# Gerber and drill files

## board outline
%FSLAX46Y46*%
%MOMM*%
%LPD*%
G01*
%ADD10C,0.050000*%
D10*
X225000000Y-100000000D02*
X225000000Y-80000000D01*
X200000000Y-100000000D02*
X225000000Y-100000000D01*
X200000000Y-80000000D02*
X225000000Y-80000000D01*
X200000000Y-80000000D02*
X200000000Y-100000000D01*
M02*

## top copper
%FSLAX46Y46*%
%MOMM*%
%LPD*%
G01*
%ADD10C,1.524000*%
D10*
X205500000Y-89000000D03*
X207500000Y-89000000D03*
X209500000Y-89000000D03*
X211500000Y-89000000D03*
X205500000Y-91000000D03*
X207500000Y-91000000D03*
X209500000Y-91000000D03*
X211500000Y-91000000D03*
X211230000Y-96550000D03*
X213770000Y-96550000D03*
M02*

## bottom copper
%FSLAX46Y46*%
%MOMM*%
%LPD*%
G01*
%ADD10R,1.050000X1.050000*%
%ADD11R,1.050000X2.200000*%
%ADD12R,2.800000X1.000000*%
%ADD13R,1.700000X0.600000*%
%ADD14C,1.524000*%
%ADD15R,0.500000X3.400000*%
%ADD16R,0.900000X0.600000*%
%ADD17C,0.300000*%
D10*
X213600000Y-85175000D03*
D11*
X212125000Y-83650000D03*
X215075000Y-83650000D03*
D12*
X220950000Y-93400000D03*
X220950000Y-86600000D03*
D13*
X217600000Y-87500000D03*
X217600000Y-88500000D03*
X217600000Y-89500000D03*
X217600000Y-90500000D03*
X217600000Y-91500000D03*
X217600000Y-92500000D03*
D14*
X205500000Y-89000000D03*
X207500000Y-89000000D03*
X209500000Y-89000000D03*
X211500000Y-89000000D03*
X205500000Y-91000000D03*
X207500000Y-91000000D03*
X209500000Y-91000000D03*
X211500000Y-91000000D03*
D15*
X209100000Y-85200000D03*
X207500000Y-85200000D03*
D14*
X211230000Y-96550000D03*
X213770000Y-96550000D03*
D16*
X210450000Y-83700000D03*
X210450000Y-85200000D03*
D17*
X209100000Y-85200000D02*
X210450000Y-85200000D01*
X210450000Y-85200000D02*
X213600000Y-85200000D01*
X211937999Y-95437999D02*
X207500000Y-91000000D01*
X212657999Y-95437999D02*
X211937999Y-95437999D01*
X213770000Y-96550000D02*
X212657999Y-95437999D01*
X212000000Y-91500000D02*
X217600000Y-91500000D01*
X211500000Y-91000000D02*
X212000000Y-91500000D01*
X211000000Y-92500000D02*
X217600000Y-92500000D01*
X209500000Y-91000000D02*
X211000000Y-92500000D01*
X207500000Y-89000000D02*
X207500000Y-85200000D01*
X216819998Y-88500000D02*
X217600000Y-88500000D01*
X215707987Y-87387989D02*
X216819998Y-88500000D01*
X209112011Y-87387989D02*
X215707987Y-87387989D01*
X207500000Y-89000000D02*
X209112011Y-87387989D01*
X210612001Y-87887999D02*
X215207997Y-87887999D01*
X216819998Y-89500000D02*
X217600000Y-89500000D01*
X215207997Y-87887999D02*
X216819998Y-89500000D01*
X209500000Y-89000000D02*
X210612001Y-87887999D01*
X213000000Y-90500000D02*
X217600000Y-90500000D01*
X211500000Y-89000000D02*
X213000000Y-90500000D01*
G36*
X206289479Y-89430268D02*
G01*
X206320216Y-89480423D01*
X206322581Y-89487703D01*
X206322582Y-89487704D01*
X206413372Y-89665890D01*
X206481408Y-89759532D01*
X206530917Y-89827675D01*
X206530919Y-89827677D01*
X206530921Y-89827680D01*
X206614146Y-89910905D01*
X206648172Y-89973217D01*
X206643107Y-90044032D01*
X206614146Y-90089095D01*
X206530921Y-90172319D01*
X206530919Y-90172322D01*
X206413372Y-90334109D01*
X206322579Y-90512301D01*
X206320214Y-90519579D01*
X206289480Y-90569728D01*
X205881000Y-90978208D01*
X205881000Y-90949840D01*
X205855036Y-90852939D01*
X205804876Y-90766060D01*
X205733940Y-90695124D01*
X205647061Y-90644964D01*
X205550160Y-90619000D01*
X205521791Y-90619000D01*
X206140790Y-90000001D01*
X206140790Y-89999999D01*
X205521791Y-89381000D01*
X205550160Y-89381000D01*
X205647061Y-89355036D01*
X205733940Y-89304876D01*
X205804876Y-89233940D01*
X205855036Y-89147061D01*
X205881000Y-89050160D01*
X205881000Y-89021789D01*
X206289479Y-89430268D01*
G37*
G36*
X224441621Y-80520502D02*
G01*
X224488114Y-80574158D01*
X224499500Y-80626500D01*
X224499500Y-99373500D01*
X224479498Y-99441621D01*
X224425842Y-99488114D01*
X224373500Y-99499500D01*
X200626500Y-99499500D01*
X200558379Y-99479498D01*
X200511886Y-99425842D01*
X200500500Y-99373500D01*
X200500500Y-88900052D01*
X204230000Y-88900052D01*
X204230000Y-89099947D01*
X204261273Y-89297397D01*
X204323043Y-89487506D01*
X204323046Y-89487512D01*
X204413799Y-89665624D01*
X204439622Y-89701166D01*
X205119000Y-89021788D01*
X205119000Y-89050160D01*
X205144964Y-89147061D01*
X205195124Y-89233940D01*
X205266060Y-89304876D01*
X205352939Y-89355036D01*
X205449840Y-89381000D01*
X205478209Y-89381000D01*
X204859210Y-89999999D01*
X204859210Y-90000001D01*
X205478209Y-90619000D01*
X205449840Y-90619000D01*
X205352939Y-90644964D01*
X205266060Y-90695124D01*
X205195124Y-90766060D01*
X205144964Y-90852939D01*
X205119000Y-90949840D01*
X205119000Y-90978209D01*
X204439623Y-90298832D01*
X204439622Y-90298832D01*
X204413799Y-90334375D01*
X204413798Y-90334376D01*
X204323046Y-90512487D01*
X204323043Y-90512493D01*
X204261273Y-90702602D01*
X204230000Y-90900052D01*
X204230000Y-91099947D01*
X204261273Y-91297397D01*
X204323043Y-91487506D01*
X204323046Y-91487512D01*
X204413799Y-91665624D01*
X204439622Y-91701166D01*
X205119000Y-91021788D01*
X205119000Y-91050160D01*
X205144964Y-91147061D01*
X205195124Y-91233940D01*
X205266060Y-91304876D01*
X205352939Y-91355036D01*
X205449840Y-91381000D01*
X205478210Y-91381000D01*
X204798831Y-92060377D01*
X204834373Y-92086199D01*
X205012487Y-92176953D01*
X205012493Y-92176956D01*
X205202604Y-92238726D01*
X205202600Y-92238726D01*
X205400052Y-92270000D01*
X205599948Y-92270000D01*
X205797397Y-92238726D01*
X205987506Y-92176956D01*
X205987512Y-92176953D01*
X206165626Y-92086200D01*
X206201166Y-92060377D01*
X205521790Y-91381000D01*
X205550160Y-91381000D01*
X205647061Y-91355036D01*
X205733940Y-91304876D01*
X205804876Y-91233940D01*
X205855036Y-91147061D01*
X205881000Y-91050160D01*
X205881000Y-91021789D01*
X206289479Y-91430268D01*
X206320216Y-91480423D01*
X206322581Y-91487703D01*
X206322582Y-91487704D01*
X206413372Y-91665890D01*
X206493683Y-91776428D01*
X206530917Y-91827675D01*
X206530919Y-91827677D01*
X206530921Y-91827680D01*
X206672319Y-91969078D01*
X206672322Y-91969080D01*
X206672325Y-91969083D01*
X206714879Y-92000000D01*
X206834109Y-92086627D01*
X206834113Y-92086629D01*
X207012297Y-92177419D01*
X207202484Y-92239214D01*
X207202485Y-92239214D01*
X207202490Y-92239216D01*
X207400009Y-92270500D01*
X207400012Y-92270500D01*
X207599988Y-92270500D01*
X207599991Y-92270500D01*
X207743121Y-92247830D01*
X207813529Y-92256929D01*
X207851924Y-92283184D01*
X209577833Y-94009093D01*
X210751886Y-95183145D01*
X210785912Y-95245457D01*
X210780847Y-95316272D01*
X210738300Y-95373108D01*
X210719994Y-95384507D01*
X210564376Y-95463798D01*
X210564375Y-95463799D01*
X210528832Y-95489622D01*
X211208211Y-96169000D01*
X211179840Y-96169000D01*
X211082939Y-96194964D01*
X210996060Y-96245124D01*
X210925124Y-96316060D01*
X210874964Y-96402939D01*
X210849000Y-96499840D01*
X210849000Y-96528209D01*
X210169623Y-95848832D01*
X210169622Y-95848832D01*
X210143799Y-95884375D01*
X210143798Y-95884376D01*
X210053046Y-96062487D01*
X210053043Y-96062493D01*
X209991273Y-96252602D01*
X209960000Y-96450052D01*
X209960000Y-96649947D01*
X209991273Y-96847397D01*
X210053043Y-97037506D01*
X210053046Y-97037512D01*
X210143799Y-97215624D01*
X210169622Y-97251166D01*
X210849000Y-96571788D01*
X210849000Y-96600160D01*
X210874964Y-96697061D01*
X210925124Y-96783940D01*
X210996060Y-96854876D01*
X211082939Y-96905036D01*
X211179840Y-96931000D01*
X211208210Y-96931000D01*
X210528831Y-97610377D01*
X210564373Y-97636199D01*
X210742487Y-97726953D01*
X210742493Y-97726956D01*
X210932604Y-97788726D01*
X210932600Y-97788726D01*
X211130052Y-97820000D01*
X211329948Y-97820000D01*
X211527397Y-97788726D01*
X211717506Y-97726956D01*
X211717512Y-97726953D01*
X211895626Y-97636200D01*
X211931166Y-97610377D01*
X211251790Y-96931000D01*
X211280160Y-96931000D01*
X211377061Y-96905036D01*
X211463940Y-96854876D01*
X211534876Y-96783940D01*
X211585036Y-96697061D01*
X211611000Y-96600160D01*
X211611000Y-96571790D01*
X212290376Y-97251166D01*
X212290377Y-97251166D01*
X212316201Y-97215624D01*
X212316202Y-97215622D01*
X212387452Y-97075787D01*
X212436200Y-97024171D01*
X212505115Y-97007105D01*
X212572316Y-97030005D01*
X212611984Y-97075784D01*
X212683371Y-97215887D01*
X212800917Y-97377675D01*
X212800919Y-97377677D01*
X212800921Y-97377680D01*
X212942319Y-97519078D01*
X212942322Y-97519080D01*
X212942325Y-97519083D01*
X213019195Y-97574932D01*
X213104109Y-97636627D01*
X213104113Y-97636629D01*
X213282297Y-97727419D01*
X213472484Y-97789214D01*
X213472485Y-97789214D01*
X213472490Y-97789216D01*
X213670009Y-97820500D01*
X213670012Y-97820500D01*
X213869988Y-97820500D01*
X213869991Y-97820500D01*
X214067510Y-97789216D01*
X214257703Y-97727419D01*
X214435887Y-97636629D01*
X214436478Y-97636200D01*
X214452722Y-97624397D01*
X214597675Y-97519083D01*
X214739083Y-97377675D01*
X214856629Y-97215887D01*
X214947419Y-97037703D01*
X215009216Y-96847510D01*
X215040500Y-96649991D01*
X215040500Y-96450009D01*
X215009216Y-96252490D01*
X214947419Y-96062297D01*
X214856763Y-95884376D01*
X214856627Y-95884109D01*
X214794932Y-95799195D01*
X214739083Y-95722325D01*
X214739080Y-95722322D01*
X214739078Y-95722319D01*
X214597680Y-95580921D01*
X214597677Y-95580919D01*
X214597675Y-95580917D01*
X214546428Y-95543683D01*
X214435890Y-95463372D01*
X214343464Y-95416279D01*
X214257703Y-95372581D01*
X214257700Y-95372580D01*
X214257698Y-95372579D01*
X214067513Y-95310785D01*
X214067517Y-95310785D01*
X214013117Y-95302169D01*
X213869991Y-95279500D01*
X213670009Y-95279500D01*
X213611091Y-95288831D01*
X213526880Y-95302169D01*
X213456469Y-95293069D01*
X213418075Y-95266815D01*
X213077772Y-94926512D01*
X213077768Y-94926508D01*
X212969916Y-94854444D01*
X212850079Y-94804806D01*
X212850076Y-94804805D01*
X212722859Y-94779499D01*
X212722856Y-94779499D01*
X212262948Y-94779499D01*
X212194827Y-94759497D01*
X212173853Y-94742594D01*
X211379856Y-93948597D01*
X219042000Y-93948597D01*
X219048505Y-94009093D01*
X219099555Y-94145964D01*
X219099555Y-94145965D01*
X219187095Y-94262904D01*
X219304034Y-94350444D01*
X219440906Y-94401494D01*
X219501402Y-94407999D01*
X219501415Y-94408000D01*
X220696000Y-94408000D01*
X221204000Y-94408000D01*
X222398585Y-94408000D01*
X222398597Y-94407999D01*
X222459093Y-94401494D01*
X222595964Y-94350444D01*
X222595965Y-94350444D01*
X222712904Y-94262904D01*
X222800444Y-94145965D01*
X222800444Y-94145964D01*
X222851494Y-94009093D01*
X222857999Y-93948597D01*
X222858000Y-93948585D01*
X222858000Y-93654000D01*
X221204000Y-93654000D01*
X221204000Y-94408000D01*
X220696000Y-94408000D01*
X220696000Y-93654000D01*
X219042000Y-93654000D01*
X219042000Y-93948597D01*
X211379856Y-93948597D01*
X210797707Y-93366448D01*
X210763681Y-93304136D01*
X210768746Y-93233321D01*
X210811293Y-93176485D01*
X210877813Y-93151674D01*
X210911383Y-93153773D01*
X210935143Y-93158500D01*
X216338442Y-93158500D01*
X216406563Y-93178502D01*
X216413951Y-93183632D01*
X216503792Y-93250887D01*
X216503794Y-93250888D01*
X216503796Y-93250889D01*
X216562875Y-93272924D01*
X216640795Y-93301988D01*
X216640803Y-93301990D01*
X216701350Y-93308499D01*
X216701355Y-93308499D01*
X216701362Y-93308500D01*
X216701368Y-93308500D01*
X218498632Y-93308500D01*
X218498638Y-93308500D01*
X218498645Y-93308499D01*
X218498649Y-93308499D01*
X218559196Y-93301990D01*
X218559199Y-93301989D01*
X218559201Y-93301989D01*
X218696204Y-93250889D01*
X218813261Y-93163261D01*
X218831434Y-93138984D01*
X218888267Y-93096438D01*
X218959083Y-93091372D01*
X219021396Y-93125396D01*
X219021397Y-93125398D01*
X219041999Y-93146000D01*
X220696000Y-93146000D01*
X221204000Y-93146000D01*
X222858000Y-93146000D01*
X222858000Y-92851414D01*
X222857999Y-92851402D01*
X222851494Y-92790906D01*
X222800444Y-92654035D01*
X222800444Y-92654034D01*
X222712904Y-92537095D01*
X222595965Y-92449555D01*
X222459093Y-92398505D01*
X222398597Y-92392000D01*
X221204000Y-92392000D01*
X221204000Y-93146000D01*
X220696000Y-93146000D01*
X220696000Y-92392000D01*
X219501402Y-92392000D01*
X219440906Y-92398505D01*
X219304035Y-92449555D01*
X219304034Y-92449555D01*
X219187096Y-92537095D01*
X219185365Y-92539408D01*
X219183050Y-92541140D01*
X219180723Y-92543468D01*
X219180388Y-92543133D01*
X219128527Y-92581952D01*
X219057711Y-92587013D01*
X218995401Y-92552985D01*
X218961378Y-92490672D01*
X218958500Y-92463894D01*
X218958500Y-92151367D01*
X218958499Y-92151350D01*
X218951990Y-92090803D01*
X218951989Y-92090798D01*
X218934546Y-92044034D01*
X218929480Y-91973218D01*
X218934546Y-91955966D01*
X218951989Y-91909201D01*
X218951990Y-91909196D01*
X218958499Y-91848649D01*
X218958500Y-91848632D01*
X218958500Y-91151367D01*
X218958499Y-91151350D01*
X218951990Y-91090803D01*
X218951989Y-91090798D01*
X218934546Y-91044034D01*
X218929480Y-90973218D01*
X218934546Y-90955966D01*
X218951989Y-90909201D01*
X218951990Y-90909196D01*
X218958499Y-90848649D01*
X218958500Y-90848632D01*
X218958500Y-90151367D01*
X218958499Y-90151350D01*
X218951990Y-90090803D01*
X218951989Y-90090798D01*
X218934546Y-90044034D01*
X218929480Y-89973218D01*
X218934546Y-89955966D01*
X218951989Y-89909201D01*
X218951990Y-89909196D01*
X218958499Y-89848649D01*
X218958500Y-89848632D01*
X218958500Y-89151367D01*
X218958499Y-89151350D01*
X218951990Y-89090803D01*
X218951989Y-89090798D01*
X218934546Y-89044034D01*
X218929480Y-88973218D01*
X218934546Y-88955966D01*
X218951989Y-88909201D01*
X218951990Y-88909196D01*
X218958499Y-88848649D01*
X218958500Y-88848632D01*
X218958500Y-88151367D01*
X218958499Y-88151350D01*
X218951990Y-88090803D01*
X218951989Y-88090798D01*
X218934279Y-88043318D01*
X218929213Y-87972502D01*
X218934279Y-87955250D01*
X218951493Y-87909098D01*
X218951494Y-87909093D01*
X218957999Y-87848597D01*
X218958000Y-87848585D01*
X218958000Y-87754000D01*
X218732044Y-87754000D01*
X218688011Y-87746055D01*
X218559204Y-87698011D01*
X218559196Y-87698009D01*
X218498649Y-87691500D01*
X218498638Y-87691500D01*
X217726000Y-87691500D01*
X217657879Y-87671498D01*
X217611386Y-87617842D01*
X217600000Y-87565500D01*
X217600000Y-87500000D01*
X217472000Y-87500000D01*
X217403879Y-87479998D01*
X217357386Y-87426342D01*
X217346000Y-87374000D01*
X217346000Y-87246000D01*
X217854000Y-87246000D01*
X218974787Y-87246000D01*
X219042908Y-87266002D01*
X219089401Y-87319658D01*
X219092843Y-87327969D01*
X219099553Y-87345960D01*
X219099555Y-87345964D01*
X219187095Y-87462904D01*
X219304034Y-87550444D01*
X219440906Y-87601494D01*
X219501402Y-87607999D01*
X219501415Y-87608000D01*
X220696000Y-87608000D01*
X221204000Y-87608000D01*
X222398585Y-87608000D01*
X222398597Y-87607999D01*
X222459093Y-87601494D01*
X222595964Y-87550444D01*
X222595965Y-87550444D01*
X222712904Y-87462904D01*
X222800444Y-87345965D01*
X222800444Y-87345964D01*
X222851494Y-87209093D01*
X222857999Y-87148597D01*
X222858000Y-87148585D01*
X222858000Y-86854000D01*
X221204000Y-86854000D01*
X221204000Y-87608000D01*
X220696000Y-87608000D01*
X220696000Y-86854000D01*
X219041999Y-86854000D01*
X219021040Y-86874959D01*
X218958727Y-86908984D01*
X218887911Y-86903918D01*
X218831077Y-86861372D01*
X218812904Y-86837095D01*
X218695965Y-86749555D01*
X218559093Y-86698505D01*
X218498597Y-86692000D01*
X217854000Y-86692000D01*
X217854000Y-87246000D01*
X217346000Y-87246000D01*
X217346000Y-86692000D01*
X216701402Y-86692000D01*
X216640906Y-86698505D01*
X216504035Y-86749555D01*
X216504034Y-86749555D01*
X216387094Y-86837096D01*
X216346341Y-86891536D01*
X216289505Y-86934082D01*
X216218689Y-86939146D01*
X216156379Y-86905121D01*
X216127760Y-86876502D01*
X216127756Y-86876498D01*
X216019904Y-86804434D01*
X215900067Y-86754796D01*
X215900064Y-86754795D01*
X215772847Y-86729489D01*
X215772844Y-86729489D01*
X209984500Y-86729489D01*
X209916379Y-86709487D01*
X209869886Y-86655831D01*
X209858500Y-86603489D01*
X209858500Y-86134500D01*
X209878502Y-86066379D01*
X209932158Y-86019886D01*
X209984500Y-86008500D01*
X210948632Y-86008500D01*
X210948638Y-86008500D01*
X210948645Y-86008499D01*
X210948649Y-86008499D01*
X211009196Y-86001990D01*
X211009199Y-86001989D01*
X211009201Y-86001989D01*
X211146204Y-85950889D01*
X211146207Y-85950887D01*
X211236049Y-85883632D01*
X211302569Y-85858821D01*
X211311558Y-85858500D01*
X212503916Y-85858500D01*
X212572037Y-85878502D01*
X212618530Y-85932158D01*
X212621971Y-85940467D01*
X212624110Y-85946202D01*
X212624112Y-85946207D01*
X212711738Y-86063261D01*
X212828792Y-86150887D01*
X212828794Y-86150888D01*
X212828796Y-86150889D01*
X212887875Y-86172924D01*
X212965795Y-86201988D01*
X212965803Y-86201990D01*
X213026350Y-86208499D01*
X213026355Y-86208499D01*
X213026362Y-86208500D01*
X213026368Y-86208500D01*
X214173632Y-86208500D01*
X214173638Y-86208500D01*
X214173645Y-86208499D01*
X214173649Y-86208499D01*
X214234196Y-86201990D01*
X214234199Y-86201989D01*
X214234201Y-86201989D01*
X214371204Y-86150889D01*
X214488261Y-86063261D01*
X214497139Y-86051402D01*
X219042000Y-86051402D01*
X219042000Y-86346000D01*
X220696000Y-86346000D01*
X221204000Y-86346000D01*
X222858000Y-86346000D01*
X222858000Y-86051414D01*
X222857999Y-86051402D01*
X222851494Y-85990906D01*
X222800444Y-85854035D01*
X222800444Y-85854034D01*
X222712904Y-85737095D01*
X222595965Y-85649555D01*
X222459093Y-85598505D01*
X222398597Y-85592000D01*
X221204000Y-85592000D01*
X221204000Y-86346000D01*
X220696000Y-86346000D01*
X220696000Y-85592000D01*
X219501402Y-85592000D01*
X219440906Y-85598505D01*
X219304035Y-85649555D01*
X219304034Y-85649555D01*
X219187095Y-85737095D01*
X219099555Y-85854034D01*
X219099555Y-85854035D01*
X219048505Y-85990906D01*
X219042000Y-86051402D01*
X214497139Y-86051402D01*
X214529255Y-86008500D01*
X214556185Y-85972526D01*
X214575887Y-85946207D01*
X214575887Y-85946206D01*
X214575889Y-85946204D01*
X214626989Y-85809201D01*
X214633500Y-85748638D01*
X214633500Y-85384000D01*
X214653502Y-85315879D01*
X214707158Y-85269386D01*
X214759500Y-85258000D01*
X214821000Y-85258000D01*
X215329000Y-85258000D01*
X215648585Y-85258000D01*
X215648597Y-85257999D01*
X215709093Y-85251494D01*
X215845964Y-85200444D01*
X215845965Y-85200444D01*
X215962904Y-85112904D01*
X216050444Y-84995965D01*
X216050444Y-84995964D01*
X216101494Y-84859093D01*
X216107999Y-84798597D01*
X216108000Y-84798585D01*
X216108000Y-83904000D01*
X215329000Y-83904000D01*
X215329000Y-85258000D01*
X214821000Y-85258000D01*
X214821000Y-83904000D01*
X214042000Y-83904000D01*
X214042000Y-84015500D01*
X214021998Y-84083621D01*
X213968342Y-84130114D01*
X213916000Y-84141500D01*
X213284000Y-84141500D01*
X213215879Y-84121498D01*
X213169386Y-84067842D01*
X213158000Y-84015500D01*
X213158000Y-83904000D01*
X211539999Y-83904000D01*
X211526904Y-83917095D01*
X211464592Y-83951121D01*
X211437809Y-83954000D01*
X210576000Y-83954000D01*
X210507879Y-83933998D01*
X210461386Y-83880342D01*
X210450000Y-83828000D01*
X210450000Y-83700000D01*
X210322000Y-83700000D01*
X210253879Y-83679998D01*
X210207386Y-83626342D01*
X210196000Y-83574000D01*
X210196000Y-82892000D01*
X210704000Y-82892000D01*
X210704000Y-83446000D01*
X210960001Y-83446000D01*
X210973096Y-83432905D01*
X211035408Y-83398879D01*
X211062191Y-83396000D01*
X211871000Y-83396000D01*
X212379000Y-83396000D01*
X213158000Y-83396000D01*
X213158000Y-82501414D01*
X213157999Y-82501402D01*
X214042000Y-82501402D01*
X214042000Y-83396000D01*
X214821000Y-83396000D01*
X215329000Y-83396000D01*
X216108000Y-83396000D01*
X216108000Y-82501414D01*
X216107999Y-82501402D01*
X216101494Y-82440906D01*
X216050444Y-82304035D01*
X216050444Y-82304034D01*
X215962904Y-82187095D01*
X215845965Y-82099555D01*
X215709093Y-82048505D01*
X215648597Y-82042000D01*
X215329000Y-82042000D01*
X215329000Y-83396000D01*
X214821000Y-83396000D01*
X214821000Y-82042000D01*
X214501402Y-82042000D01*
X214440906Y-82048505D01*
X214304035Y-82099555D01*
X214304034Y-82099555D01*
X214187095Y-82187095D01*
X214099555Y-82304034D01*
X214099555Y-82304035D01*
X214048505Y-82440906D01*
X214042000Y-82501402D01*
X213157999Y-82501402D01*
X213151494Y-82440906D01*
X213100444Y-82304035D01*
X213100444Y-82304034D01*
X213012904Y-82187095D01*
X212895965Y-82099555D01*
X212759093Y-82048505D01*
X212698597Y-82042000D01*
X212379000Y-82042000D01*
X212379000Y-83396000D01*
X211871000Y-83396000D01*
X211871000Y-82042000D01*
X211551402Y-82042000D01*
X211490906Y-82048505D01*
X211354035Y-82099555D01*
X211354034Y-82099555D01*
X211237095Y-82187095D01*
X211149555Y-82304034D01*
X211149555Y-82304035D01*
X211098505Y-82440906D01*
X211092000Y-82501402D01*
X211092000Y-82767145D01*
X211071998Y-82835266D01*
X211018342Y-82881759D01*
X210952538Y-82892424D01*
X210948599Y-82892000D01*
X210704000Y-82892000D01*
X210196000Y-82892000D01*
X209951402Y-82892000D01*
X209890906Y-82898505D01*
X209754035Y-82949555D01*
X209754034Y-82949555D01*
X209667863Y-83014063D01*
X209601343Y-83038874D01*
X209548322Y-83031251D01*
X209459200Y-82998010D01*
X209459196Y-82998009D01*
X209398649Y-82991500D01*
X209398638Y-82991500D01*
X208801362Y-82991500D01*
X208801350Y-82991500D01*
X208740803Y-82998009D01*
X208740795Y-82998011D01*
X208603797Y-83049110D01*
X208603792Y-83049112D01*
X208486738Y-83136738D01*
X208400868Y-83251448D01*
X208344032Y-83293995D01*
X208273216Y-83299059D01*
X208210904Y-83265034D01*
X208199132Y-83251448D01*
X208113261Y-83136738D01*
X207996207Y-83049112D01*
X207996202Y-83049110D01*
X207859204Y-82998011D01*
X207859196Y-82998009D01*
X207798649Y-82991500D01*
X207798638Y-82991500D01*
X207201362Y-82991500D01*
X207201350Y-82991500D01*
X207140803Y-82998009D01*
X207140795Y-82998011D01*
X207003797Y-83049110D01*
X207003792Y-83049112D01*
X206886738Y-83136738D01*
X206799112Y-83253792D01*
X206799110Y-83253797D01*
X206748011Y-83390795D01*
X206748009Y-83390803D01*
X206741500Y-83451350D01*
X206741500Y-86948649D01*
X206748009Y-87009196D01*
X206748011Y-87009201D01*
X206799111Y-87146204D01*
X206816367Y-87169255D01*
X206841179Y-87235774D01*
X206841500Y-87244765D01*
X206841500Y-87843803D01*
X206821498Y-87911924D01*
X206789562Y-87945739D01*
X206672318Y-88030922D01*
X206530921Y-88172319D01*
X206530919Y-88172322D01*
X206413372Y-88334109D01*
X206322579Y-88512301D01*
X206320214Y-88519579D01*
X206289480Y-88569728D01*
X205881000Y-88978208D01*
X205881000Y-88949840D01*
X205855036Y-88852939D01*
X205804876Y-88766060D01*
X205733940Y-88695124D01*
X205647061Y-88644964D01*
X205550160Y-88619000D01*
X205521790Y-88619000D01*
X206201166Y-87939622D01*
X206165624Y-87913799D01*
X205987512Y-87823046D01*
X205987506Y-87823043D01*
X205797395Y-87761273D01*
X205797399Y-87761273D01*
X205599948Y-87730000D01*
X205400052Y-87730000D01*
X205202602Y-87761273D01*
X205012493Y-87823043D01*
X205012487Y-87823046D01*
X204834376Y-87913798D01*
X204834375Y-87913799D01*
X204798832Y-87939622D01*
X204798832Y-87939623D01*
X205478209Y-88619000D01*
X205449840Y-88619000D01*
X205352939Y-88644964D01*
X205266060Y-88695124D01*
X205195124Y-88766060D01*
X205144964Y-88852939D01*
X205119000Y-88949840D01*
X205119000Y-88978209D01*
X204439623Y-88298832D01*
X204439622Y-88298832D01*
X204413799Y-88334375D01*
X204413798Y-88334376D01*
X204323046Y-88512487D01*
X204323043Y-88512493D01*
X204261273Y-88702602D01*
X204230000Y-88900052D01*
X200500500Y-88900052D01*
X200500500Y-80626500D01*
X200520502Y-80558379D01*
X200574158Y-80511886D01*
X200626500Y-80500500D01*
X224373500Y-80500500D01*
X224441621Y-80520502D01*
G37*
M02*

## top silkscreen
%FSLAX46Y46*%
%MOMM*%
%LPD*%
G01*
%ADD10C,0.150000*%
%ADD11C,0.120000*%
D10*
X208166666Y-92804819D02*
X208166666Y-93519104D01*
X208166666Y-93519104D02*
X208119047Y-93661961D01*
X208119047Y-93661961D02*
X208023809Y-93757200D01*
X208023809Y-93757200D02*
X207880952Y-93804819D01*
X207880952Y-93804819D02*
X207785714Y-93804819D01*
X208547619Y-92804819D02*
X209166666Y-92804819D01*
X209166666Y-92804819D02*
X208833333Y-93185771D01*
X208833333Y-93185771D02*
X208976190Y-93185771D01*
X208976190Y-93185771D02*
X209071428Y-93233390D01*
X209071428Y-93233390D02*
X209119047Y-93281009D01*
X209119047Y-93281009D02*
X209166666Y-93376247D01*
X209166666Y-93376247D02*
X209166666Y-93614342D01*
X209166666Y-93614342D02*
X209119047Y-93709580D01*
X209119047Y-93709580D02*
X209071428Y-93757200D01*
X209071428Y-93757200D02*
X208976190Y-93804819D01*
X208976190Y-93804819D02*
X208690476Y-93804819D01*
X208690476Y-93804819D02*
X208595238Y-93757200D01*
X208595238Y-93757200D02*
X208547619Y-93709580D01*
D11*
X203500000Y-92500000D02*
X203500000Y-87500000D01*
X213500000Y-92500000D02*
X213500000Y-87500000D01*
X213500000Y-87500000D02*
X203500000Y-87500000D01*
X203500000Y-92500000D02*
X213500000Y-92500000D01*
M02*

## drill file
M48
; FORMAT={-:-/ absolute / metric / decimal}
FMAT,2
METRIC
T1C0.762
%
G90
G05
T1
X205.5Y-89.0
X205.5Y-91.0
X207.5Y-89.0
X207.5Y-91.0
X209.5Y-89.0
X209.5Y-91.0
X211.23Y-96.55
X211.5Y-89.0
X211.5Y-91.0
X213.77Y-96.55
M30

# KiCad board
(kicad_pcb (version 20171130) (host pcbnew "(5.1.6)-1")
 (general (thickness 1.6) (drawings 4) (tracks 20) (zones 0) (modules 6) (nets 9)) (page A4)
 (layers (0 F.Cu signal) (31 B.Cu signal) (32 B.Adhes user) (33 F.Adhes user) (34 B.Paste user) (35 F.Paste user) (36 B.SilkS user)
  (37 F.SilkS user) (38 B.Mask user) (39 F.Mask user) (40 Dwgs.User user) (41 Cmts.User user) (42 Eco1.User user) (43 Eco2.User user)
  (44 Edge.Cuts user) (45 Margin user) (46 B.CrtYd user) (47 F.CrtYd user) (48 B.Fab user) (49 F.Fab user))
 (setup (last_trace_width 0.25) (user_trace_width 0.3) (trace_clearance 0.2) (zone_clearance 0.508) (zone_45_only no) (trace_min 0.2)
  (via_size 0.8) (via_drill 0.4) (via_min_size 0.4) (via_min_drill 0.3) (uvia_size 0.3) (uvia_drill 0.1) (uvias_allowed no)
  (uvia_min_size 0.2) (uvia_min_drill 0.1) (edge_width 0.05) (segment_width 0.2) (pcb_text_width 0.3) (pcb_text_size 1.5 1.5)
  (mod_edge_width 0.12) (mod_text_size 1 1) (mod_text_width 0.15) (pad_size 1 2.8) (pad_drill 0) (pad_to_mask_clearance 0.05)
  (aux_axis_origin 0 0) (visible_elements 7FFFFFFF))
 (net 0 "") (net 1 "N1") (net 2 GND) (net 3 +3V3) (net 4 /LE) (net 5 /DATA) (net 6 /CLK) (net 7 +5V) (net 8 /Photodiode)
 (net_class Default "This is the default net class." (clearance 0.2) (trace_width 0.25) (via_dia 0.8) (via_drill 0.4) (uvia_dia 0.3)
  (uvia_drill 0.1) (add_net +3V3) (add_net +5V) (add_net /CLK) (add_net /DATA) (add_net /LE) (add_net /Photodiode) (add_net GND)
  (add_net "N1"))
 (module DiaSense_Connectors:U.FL (layer B.Cu) (at 213.6 83.65 180)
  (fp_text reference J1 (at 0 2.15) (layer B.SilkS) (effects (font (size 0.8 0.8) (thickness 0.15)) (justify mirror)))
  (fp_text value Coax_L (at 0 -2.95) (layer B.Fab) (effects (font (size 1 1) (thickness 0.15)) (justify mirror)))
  (pad 1 smd rect (at 0 -1.525 180) (size 1.05 1.05) (layers B.Cu B.Paste B.Mask) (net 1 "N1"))
  (pad 2 smd rect (at 1.475 0 180) (size 1.05 2.2) (layers B.Cu B.Paste B.Mask) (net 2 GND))
  (pad 2 smd rect (at -1.475 0 180) (size 1.05 2.2) (layers B.Cu B.Paste B.Mask) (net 2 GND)))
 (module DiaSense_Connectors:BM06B (layer B.Cu) (at 218.45 90 90)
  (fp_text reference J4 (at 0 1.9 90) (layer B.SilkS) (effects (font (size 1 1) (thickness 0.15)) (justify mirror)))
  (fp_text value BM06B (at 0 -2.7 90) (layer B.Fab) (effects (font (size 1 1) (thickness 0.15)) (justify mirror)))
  (pad "" smd rect (at -3.4 2.5 90) (size 1 2.8) (layers B.Cu B.Paste B.Mask) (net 2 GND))
  (pad "" smd rect (at 3.4 2.5 90) (size 1 2.8) (layers B.Cu B.Paste B.Mask) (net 2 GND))
  (pad 6 smd rect (at 2.5 -0.85 90) (size 0.6 1.7) (layers B.Cu B.Paste B.Mask) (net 2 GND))
  (pad 5 smd rect (at 1.5 -0.85 90) (size 0.6 1.7) (layers B.Cu B.Paste B.Mask) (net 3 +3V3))
  (pad 4 smd rect (at 0.5 -0.85 90) (size 0.6 1.7) (layers B.Cu B.Paste B.Mask) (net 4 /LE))
  (pad 3 smd rect (at -0.5 -0.85 90) (size 0.6 1.7) (layers B.Cu B.Paste B.Mask) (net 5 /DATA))
  (pad 2 smd rect (at -1.5 -0.85 90) (size 0.6 1.7) (layers B.Cu B.Paste B.Mask) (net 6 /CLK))
  (pad 1 smd rect (at -2.5 -0.85 90) (size 0.6 1.7) (layers B.Cu B.Paste B.Mask) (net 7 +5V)))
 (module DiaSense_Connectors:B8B (layer F.Cu) (at 208.5 90 180)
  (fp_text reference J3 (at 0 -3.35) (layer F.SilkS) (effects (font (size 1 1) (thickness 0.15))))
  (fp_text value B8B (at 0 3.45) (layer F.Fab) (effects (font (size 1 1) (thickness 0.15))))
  (fp_line (start 5 -2.5) (end 5 2.5) (layer F.SilkS) (width 0.12))
  (fp_line (start -5 -2.5) (end -5 2.5) (layer F.SilkS) (width 0.12))
  (fp_line (start -5 2.5) (end 5 2.5) (layer F.SilkS) (width 0.12))
  (fp_line (start 5 -2.5) (end -5 -2.5) (layer F.SilkS) (width 0.12))
  (pad 8 thru_hole circle (at 3 1 180) (size 1.524 1.524) (drill 0.762) (layers *.Cu *.Mask) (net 2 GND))
  (pad 7 thru_hole circle (at 1 1 180) (size 1.524 1.524) (drill 0.762) (layers *.Cu *.Mask) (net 3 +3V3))
  (pad 6 thru_hole circle (at -1 1 180) (size 1.524 1.524) (drill 0.762) (layers *.Cu *.Mask) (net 4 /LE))
  (pad 5 thru_hole circle (at -3 1 180) (size 1.524 1.524) (drill 0.762) (layers *.Cu *.Mask) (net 5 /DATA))
  (pad 4 thru_hole circle (at 3 -1 180) (size 1.524 1.524) (drill 0.762) (layers *.Cu *.Mask) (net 2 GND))
  (pad 3 thru_hole circle (at 1 -1 180) (size 1.524 1.524) (drill 0.762) (layers *.Cu *.Mask) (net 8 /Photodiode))
  (pad 2 thru_hole circle (at -1 -1 180) (size 1.524 1.524) (drill 0.762) (layers *.Cu *.Mask) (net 7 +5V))
  (pad 1 thru_hole circle (at -3 -1 180) (size 1.524 1.524) (drill 0.762) (layers *.Cu *.Mask) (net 6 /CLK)))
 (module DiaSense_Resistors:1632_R (layer B.Cu) (at 208.3 85.2 270)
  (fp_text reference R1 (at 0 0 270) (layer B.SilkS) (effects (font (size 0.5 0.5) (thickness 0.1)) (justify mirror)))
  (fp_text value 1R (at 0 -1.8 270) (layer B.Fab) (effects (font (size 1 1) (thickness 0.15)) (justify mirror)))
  (pad 2 smd rect (at 0 -0.8 90) (size 3.4 0.5) (layers B.Cu B.Paste B.Mask) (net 1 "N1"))
  (pad 1 smd rect (at 0 0.8 90) (size 3.4 0.5) (layers B.Cu B.Paste B.Mask) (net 3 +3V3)))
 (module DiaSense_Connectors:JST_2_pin (layer B.Cu) (at 212.5 96.55 180)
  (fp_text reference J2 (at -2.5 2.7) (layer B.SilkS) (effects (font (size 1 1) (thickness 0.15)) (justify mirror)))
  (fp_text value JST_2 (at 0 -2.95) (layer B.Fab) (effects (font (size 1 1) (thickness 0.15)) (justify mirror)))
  (pad 2 thru_hole circle (at 1.27 0 180) (size 1.524 1.524) (drill 0.762) (layers *.Cu *.Mask) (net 2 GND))
  (pad 1 thru_hole circle (at -1.27 0 180) (size 1.524 1.524) (drill 0.762) (layers *.Cu *.Mask) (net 8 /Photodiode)))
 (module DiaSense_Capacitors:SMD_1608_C (layer B.Cu) (at 210.45 84.45)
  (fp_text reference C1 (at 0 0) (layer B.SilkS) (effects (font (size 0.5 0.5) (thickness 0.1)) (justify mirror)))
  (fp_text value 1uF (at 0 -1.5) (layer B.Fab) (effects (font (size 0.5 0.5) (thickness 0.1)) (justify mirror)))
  (pad 2 smd rect (at 0 -0.75) (size 0.9 0.6) (layers B.Cu B.Paste B.Mask) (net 2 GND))
  (pad 1 smd rect (at 0 0.75) (size 0.9 0.6) (layers B.Cu B.Paste B.Mask) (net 1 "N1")))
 (gr_line (start 225 100) (end 225 80) (layer Edge.Cuts) (width 0.05))
 (gr_line (start 200 100) (end 225 100) (layer Edge.Cuts) (width 0.05))
 (gr_line (start 200 80) (end 225 80) (layer Edge.Cuts) (width 0.05))
 (gr_line (start 200 80) (end 200 100) (layer Edge.Cuts) (width 0.05))
 (segment (start 209.1 85.2) (end 210.45 85.2) (width 0.3) (layer B.Cu) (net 1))
 (segment (start 210.45 85.2) (end 213.6 85.2) (width 0.3) (layer B.Cu) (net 1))
 (segment (start 211.937999 95.437999) (end 207.5 91) (width 0.3) (layer B.Cu) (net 8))
 (segment (start 212.657999 95.437999) (end 211.937999 95.437999) (width 0.3) (layer B.Cu) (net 8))
 (segment (start 213.77 96.55) (end 212.657999 95.437999) (width 0.3) (layer B.Cu) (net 8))
 (segment (start 212 91.5) (end 217.6 91.5) (width 0.3) (layer B.Cu) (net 6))
 (segment (start 211.5 91) (end 212 91.5) (width 0.3) (layer B.Cu) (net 6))
 (segment (start 211 92.5) (end 217.6 92.5) (width 0.3) (layer B.Cu) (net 7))
 (segment (start 209.5 91) (end 211 92.5) (width 0.3) (layer B.Cu) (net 7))
 (segment (start 207.5 89) (end 207.5 85.2) (width 0.3) (layer B.Cu) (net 3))
 (segment (start 216.819998 88.5) (end 217.6 88.5) (width 0.3) (layer B.Cu) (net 3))
 (segment (start 215.707987 87.387989) (end 216.819998 88.5) (width 0.3) (layer B.Cu) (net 3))
 (segment (start 209.112011 87.387989) (end 215.707987 87.387989) (width 0.3) (layer B.Cu) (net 3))
 (segment (start 207.5 89) (end 209.112011 87.387989) (width 0.3) (layer B.Cu) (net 3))
 (segment (start 210.612001 87.887999) (end 215.207997 87.887999) (width 0.3) (layer B.Cu) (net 4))
 (segment (start 216.819998 89.5) (end 217.6 89.5) (width 0.3) (layer B.Cu) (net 4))
 (segment (start 215.207997 87.887999) (end 216.819998 89.5) (width 0.3) (layer B.Cu) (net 4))
 (segment (start 209.5 89) (end 210.612001 87.887999) (width 0.3) (layer B.Cu) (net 4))
 (segment (start 213 90.5) (end 217.6 90.5) (width 0.3) (layer B.Cu) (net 5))
 (segment (start 211.5 89) (end 213 90.5) (width 0.3) (layer B.Cu) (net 5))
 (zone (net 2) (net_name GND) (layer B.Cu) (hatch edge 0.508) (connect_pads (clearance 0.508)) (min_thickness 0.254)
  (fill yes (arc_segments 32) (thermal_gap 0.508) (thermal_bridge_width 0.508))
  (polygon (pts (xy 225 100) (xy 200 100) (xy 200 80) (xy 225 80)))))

